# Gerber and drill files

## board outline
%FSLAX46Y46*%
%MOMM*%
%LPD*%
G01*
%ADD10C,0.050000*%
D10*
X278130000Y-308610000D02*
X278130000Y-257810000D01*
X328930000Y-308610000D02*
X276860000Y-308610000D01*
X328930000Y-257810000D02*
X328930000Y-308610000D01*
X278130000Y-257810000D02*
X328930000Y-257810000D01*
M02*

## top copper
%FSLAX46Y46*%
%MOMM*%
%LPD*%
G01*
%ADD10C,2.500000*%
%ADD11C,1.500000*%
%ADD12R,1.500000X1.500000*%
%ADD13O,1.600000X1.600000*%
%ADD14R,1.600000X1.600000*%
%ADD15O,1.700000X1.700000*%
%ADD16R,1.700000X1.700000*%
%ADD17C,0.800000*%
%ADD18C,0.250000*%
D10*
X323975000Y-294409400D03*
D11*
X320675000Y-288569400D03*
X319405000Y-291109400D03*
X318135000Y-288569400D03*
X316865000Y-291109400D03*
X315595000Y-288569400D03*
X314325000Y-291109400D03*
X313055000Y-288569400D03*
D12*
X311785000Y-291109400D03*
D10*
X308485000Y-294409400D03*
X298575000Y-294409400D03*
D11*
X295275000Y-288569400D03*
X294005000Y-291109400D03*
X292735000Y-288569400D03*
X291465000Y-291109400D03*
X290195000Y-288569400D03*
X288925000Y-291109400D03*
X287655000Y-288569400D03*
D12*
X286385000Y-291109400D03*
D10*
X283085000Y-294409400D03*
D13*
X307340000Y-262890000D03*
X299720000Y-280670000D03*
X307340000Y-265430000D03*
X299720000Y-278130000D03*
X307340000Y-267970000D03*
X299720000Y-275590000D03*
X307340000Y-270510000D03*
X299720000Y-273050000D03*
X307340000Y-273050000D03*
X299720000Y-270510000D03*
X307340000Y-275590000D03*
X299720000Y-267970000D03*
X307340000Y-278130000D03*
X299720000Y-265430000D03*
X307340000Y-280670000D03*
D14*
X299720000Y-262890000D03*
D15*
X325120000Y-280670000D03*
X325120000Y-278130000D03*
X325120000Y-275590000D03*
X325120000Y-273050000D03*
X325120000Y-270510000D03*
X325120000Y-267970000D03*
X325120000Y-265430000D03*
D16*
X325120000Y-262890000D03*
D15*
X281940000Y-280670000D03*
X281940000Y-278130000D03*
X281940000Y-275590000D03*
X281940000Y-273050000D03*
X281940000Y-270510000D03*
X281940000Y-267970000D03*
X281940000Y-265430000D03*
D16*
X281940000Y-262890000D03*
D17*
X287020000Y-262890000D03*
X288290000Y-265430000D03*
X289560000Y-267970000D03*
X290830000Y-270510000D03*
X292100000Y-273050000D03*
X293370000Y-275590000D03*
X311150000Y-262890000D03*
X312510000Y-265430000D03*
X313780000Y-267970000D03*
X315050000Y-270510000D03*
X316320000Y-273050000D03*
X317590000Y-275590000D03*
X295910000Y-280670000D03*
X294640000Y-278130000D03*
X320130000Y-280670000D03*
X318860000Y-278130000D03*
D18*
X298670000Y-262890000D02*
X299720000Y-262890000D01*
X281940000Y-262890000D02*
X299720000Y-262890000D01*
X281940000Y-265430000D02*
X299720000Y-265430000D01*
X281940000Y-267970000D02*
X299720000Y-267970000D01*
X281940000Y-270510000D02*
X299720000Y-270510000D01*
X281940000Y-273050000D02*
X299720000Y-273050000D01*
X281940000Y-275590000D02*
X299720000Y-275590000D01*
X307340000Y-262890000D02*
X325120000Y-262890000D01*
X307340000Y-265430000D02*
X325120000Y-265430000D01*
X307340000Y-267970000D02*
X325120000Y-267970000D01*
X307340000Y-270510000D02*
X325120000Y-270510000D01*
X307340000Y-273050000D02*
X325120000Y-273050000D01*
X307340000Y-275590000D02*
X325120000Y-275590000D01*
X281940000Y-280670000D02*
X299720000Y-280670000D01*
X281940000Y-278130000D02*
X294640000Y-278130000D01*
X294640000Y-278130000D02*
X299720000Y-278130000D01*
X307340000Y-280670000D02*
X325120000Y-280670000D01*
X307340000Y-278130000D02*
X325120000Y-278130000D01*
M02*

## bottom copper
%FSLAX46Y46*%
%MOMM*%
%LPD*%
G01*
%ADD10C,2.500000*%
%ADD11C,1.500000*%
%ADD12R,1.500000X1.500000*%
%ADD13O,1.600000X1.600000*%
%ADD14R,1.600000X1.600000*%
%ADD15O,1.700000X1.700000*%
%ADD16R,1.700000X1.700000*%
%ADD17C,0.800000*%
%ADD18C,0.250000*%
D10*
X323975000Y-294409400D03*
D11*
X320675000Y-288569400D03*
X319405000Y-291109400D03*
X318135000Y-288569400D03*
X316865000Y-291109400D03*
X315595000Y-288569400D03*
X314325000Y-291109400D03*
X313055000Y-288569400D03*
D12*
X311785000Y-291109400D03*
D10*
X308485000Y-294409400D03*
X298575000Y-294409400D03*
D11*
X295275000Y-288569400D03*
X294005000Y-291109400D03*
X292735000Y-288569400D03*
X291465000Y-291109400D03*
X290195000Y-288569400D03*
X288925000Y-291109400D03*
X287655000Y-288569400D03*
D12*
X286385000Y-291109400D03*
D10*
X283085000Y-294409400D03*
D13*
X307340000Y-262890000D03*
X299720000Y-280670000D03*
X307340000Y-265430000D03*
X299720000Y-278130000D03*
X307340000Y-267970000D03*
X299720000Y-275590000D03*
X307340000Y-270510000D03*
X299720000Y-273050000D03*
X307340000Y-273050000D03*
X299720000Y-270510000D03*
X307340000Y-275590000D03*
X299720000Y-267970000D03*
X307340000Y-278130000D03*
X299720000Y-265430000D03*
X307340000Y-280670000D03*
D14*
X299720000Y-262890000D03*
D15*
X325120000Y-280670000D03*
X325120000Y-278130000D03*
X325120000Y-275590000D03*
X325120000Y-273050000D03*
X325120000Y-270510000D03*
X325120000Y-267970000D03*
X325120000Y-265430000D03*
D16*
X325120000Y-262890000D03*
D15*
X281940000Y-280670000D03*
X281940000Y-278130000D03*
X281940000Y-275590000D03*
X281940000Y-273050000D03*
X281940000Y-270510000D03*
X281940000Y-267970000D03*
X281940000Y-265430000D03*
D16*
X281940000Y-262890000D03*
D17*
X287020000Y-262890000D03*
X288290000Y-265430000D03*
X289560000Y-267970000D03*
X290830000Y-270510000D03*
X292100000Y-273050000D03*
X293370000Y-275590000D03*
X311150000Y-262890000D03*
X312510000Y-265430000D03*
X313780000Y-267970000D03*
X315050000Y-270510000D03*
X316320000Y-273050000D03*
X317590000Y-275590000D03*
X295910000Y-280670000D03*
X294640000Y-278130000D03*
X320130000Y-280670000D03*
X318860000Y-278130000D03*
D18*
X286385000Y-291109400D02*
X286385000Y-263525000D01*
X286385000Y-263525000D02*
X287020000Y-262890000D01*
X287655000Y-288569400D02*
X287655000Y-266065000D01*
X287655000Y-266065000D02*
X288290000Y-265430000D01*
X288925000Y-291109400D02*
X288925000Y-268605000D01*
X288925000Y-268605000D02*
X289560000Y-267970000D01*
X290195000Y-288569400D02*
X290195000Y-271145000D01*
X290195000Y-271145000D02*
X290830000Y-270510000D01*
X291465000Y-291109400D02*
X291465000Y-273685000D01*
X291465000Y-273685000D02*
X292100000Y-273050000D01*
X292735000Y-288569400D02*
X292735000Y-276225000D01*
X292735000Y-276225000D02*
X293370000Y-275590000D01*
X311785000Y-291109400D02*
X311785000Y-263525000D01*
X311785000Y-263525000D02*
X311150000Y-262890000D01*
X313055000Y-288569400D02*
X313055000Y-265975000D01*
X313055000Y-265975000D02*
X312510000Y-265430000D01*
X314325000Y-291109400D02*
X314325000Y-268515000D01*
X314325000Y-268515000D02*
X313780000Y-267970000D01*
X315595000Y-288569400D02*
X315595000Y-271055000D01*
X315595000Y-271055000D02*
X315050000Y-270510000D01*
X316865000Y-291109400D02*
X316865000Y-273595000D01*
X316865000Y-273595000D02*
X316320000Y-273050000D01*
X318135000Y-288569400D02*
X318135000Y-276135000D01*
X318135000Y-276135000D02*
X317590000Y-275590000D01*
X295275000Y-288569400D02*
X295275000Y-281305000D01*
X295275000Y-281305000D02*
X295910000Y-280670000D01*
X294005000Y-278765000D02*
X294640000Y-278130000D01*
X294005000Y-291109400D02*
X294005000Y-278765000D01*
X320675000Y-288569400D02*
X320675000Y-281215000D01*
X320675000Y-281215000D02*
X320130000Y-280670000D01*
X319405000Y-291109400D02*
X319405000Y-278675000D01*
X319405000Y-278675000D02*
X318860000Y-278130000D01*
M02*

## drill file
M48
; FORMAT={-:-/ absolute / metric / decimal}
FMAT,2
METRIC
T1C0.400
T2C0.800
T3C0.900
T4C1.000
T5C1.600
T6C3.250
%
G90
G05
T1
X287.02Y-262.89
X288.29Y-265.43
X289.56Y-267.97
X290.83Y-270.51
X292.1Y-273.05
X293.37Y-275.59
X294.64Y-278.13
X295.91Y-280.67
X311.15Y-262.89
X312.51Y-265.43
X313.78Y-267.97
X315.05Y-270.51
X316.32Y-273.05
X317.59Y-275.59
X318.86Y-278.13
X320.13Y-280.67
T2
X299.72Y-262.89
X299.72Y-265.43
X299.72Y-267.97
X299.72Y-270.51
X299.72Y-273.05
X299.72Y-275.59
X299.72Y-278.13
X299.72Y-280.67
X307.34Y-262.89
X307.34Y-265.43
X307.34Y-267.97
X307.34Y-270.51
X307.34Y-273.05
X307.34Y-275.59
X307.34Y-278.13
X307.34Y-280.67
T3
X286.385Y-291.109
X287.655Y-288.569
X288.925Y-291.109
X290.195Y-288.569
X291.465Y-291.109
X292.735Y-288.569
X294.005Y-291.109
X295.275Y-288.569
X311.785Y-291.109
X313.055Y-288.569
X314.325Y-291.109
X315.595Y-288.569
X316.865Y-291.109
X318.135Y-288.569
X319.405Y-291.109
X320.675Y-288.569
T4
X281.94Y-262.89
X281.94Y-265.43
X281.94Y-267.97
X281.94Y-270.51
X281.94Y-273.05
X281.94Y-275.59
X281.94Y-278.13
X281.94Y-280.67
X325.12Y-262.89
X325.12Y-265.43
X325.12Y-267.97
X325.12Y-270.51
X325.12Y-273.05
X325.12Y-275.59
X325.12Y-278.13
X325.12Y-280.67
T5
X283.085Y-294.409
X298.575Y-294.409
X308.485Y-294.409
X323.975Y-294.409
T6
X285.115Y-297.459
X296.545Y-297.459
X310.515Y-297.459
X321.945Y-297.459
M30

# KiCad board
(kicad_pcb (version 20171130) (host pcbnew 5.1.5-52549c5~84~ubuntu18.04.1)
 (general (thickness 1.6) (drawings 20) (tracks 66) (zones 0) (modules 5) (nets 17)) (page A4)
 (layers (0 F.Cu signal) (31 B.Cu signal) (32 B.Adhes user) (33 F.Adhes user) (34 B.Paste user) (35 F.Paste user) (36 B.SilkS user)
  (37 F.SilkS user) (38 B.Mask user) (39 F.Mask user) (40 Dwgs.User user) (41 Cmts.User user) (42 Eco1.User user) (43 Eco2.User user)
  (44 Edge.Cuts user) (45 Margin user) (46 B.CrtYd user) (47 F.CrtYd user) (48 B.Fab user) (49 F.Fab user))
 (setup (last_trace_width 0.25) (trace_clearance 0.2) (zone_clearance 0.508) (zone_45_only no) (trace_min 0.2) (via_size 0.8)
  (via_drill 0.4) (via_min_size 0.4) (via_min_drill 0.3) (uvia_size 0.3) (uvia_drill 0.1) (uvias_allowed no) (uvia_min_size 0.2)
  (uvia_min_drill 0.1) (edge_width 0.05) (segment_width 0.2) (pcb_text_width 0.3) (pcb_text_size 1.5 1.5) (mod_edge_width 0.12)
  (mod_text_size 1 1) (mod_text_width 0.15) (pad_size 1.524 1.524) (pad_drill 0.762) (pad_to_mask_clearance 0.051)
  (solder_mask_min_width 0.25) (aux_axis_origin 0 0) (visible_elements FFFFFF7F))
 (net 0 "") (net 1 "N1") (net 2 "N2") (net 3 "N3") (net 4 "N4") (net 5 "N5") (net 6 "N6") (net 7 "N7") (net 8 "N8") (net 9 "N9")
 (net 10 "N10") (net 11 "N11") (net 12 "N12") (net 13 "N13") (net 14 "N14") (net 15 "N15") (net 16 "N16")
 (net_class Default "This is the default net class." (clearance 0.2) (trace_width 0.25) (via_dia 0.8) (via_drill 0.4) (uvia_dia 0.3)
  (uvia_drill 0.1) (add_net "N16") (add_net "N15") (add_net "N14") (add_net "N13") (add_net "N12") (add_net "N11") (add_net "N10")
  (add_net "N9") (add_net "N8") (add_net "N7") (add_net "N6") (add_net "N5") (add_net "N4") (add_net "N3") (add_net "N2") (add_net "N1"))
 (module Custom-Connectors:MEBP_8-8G (layer F.Cu) (at 316.23 306.07 180)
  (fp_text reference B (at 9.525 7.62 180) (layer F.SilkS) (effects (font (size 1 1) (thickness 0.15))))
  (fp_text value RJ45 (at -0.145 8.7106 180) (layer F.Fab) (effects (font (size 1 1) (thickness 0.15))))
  (pad 9 thru_hole circle (at -7.745 11.6606) (size 2.5 2.5) (drill 1.6) (layers *.Cu *.Mask))
  (pad 8 thru_hole circle (at -4.445 17.5006) (size 1.5 1.5) (drill 0.9) (layers *.Cu *.Mask) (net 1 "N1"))
  (pad 7 thru_hole circle (at -3.175 14.9606) (size 1.5 1.5) (drill 0.9) (layers *.Cu *.Mask) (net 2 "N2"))
  (pad 6 thru_hole circle (at -1.905 17.5006) (size 1.5 1.5) (drill 0.9) (layers *.Cu *.Mask) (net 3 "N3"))
  (pad 5 thru_hole circle (at -0.635 14.9606) (size 1.5 1.5) (drill 0.9) (layers *.Cu *.Mask) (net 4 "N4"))
  (pad 4 thru_hole circle (at 0.635 17.5006) (size 1.5 1.5) (drill 0.9) (layers *.Cu *.Mask) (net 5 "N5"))
  (pad 3 thru_hole circle (at 1.905 14.9606) (size 1.5 1.5) (drill 0.9) (layers *.Cu *.Mask) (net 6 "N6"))
  (pad 2 thru_hole circle (at 3.175 17.5006) (size 1.5 1.5) (drill 0.9) (layers *.Cu *.Mask) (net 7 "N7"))
  (pad 1 thru_hole rect (at 4.445 14.9606) (size 1.5 1.5) (drill 0.9) (layers *.Cu *.Mask) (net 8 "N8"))
  (pad "" np_thru_hole circle (at 5.715 8.6106) (size 3.25 3.25) (drill 3.25) (layers *.Cu *.SilkS *.Mask))
  (pad "" np_thru_hole circle (at -5.715 8.6106) (size 3.25 3.25) (drill 3.25) (layers *.Cu *.SilkS *.Mask))
  (pad 9 thru_hole circle (at 7.745 11.6606) (size 2.5 2.5) (drill 1.6) (layers *.Cu *.Mask)))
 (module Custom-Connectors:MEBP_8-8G (layer F.Cu) (at 290.83 306.07 180)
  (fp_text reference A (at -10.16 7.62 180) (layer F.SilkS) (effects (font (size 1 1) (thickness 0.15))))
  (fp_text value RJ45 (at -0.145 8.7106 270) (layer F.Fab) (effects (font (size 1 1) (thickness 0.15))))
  (pad 9 thru_hole circle (at -7.745 11.6606) (size 2.5 2.5) (drill 1.6) (layers *.Cu *.Mask))
  (pad 8 thru_hole circle (at -4.445 17.5006) (size 1.5 1.5) (drill 0.9) (layers *.Cu *.Mask) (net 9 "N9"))
  (pad 7 thru_hole circle (at -3.175 14.9606) (size 1.5 1.5) (drill 0.9) (layers *.Cu *.Mask) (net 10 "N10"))
  (pad 6 thru_hole circle (at -1.905 17.5006) (size 1.5 1.5) (drill 0.9) (layers *.Cu *.Mask) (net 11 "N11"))
  (pad 5 thru_hole circle (at -0.635 14.9606) (size 1.5 1.5) (drill 0.9) (layers *.Cu *.Mask) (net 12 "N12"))
  (pad 4 thru_hole circle (at 0.635 17.5006) (size 1.5 1.5) (drill 0.9) (layers *.Cu *.Mask) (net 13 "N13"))
  (pad 3 thru_hole circle (at 1.905 14.9606) (size 1.5 1.5) (drill 0.9) (layers *.Cu *.Mask) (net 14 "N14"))
  (pad 2 thru_hole circle (at 3.175 17.5006) (size 1.5 1.5) (drill 0.9) (layers *.Cu *.Mask) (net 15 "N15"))
  (pad 1 thru_hole rect (at 4.445 14.9606) (size 1.5 1.5) (drill 0.9) (layers *.Cu *.Mask) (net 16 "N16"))
  (pad "" np_thru_hole circle (at 5.715 8.6106) (size 3.25 3.25) (drill 3.25) (layers *.Cu *.SilkS *.Mask))
  (pad "" np_thru_hole circle (at -5.715 8.6106) (size 3.25 3.25) (drill 3.25) (layers *.Cu *.SilkS *.Mask))
  (pad 9 thru_hole circle (at 7.745 11.6606) (size 2.5 2.5) (drill 1.6) (layers *.Cu *.Mask)))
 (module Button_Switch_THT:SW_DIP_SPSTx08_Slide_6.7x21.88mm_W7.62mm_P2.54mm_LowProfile (layer F.Cu) (at 299.72 262.89)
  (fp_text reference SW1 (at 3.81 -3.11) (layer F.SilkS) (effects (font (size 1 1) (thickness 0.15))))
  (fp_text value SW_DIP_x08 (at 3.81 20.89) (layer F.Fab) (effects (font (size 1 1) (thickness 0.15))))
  (pad 16 thru_hole oval (at 7.62 0) (size 1.6 1.6) (drill 0.8) (layers *.Cu *.Mask) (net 8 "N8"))
  (pad 8 thru_hole oval (at 0 17.78) (size 1.6 1.6) (drill 0.8) (layers *.Cu *.Mask) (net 9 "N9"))
  (pad 15 thru_hole oval (at 7.62 2.54) (size 1.6 1.6) (drill 0.8) (layers *.Cu *.Mask) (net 7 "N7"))
  (pad 7 thru_hole oval (at 0 15.24) (size 1.6 1.6) (drill 0.8) (layers *.Cu *.Mask) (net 10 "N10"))
  (pad 14 thru_hole oval (at 7.62 5.08) (size 1.6 1.6) (drill 0.8) (layers *.Cu *.Mask) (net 6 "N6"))
  (pad 6 thru_hole oval (at 0 12.7) (size 1.6 1.6) (drill 0.8) (layers *.Cu *.Mask) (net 11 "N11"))
  (pad 13 thru_hole oval (at 7.62 7.62) (size 1.6 1.6) (drill 0.8) (layers *.Cu *.Mask) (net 5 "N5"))
  (pad 5 thru_hole oval (at 0 10.16) (size 1.6 1.6) (drill 0.8) (layers *.Cu *.Mask) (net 12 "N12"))
  (pad 12 thru_hole oval (at 7.62 10.16) (size 1.6 1.6) (drill 0.8) (layers *.Cu *.Mask) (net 4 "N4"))
  (pad 4 thru_hole oval (at 0 7.62) (size 1.6 1.6) (drill 0.8) (layers *.Cu *.Mask) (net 13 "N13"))
  (pad 11 thru_hole oval (at 7.62 12.7) (size 1.6 1.6) (drill 0.8) (layers *.Cu *.Mask) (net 3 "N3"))
  (pad 3 thru_hole oval (at 0 5.08) (size 1.6 1.6) (drill 0.8) (layers *.Cu *.Mask) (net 14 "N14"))
  (pad 10 thru_hole oval (at 7.62 15.24) (size 1.6 1.6) (drill 0.8) (layers *.Cu *.Mask) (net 2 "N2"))
  (pad 2 thru_hole oval (at 0 2.54) (size 1.6 1.6) (drill 0.8) (layers *.Cu *.Mask) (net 15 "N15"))
  (pad 9 thru_hole oval (at 7.62 17.78) (size 1.6 1.6) (drill 0.8) (layers *.Cu *.Mask) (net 1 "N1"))
  (pad 1 thru_hole rect (at 0 0) (size 1.6 1.6) (drill 0.8) (layers *.Cu *.Mask) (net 16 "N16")))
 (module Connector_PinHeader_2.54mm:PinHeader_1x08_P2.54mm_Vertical (layer F.Cu) (at 325.12 262.89)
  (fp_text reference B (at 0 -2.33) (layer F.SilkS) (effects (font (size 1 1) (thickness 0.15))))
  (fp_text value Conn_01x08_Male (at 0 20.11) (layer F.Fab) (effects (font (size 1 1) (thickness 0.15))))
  (pad 8 thru_hole oval (at 0 17.78) (size 1.7 1.7) (drill 1) (layers *.Cu *.Mask) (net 1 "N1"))
  (pad 7 thru_hole oval (at 0 15.24) (size 1.7 1.7) (drill 1) (layers *.Cu *.Mask) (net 2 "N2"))
  (pad 6 thru_hole oval (at 0 12.7) (size 1.7 1.7) (drill 1) (layers *.Cu *.Mask) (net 3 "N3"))
  (pad 5 thru_hole oval (at 0 10.16) (size 1.7 1.7) (drill 1) (layers *.Cu *.Mask) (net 4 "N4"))
  (pad 4 thru_hole oval (at 0 7.62) (size 1.7 1.7) (drill 1) (layers *.Cu *.Mask) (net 5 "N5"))
  (pad 3 thru_hole oval (at 0 5.08) (size 1.7 1.7) (drill 1) (layers *.Cu *.Mask) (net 6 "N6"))
  (pad 2 thru_hole oval (at 0 2.54) (size 1.7 1.7) (drill 1) (layers *.Cu *.Mask) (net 7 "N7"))
  (pad 1 thru_hole rect (at 0 0) (size 1.7 1.7) (drill 1) (layers *.Cu *.Mask) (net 8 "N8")))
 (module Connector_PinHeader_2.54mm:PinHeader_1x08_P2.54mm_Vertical (layer F.Cu) (at 281.94 262.89)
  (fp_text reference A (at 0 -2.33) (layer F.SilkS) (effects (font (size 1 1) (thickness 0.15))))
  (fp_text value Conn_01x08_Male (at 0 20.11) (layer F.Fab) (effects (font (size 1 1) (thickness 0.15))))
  (pad 8 thru_hole oval (at 0 17.78) (size 1.7 1.7) (drill 1) (layers *.Cu *.Mask) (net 9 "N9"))
  (pad 7 thru_hole oval (at 0 15.24) (size 1.7 1.7) (drill 1) (layers *.Cu *.Mask) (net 10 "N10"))
  (pad 6 thru_hole oval (at 0 12.7) (size 1.7 1.7) (drill 1) (layers *.Cu *.Mask) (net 11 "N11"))
  (pad 5 thru_hole oval (at 0 10.16) (size 1.7 1.7) (drill 1) (layers *.Cu *.Mask) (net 12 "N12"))
  (pad 4 thru_hole oval (at 0 7.62) (size 1.7 1.7) (drill 1) (layers *.Cu *.Mask) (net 13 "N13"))
  (pad 3 thru_hole oval (at 0 5.08) (size 1.7 1.7) (drill 1) (layers *.Cu *.Mask) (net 14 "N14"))
  (pad 2 thru_hole oval (at 0 2.54) (size 1.7 1.7) (drill 1) (layers *.Cu *.Mask) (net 15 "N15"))
  (pad 1 thru_hole rect (at 0 0) (size 1.7 1.7) (drill 1) (layers *.Cu *.Mask) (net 16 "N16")))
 (gr_line (start 278.13 308.61) (end 278.13 257.81) (layer Edge.Cuts) (width 0.05))
 (gr_line (start 328.93 308.61) (end 276.86 308.61) (layer Edge.Cuts) (width 0.05))
 (gr_line (start 328.93 257.81) (end 328.93 308.61) (layer Edge.Cuts) (width 0.05))
 (gr_line (start 278.13 257.81) (end 328.93 257.81) (layer Edge.Cuts) (width 0.05))
 (segment (start 298.67 262.89) (end 299.72 262.89) (width 0.25) (layer F.Cu) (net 16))
 (segment (start 281.94 262.89) (end 299.72 262.89) (width 0.25) (layer F.Cu) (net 16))
 (segment (start 286.385 291.1094) (end 286.385 263.525) (width 0.25) (layer B.Cu) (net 16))
 (via (at 287.02 262.89) (size 0.8) (drill 0.4) (layers F.Cu B.Cu) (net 16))
 (segment (start 286.385 263.525) (end 287.02 262.89) (width 0.25) (layer B.Cu) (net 16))
 (segment (start 281.94 265.43) (end 299.72 265.43) (width 0.25) (layer F.Cu) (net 15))
 (via (at 288.29 265.43) (size 0.8) (drill 0.4) (layers F.Cu B.Cu) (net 15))
 (segment (start 287.655 288.5694) (end 287.655 266.065) (width 0.25) (layer B.Cu) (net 15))
 (segment (start 287.655 266.065) (end 288.29 265.43) (width 0.25) (layer B.Cu) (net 15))
 (segment (start 281.94 267.97) (end 299.72 267.97) (width 0.25) (layer F.Cu) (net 14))
 (via (at 289.56 267.97) (size 0.8) (drill 0.4) (layers F.Cu B.Cu) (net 14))
 (segment (start 288.925 291.1094) (end 288.925 268.605) (width 0.25) (layer B.Cu) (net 14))
 (segment (start 288.925 268.605) (end 289.56 267.97) (width 0.25) (layer B.Cu) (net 14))
 (segment (start 281.94 270.51) (end 299.72 270.51) (width 0.25) (layer F.Cu) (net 13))
 (via (at 290.83 270.51) (size 0.8) (drill 0.4) (layers F.Cu B.Cu) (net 13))
 (segment (start 290.195 288.5694) (end 290.195 271.145) (width 0.25) (layer B.Cu) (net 13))
 (segment (start 290.195 271.145) (end 290.83 270.51) (width 0.25) (layer B.Cu) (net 13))
 (segment (start 281.94 273.05) (end 299.72 273.05) (width 0.25) (layer F.Cu) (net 12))
 (via (at 292.1 273.05) (size 0.8) (drill 0.4) (layers F.Cu B.Cu) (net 12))
 (segment (start 291.465 291.1094) (end 291.465 273.685) (width 0.25) (layer B.Cu) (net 12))
 (segment (start 291.465 273.685) (end 292.1 273.05) (width 0.25) (layer B.Cu) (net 12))
 (segment (start 281.94 275.59) (end 299.72 275.59) (width 0.25) (layer F.Cu) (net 11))
 (via (at 293.37 275.59) (size 0.8) (drill 0.4) (layers F.Cu B.Cu) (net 11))
 (segment (start 292.735 288.5694) (end 292.735 276.225) (width 0.25) (layer B.Cu) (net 11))
 (segment (start 292.735 276.225) (end 293.37 275.59) (width 0.25) (layer B.Cu) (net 11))
 (segment (start 307.34 262.89) (end 325.12 262.89) (width 0.25) (layer F.Cu) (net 8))
 (via (at 311.15 262.89) (size 0.8) (drill 0.4) (layers F.Cu B.Cu) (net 8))
 (segment (start 311.785 291.1094) (end 311.785 263.525) (width 0.25) (layer B.Cu) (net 8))
 (segment (start 311.785 263.525) (end 311.15 262.89) (width 0.25) (layer B.Cu) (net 8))
 (segment (start 307.34 265.43) (end 325.12 265.43) (width 0.25) (layer F.Cu) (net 7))
 (via (at 312.51 265.43) (size 0.8) (drill 0.4) (layers F.Cu B.Cu) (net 7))
 (segment (start 313.055 288.5694) (end 313.055 265.975) (width 0.25) (layer B.Cu) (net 7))
 (segment (start 313.055 265.975) (end 312.51 265.43) (width 0.25) (layer B.Cu) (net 7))
 (segment (start 307.34 267.97) (end 325.12 267.97) (width 0.25) (layer F.Cu) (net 6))
 (via (at 313.78 267.97) (size 0.8) (drill 0.4) (layers F.Cu B.Cu) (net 6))
 (segment (start 314.325 291.1094) (end 314.325 268.515) (width 0.25) (layer B.Cu) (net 6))
 (segment (start 314.325 268.515) (end 313.78 267.97) (width 0.25) (layer B.Cu) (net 6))
 (segment (start 307.34 270.51) (end 325.12 270.51) (width 0.25) (layer F.Cu) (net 5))
 (via (at 315.05 270.51) (size 0.8) (drill 0.4) (layers F.Cu B.Cu) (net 5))
 (segment (start 315.595 288.5694) (end 315.595 271.055) (width 0.25) (layer B.Cu) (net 5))
 (segment (start 315.595 271.055) (end 315.05 270.51) (width 0.25) (layer B.Cu) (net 5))
 (segment (start 307.34 273.05) (end 325.12 273.05) (width 0.25) (layer F.Cu) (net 4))
 (via (at 316.32 273.05) (size 0.8) (drill 0.4) (layers F.Cu B.Cu) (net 4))
 (segment (start 316.865 291.1094) (end 316.865 273.595) (width 0.25) (layer B.Cu) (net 4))
 (segment (start 316.865 273.595) (end 316.32 273.05) (width 0.25) (layer B.Cu) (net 4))
 (segment (start 307.34 275.59) (end 325.12 275.59) (width 0.25) (layer F.Cu) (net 3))
 (via (at 317.59 275.59) (size 0.8) (drill 0.4) (layers F.Cu B.Cu) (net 3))
 (segment (start 318.135 288.5694) (end 318.135 276.135) (width 0.25) (layer B.Cu) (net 3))
 (segment (start 318.135 276.135) (end 317.59 275.59) (width 0.25) (layer B.Cu) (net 3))
 (segment (start 281.94 280.67) (end 299.72 280.67) (width 0.25) (layer F.Cu) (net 9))
 (segment (start 295.275 288.5694) (end 295.275 281.305) (width 0.25) (layer B.Cu) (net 9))
 (via (at 295.91 280.67) (size 0.8) (drill 0.4) (layers F.Cu B.Cu) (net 9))
 (segment (start 295.275 281.305) (end 295.91 280.67) (width 0.25) (layer B.Cu) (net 9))
 (via (at 294.64 278.13) (size 0.8) (drill 0.4) (layers F.Cu B.Cu) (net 10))
 (segment (start 294.005 278.765) (end 294.64 278.13) (width 0.25) (layer B.Cu) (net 10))
 (segment (start 294.005 291.1094) (end 294.005 278.765) (width 0.25) (layer B.Cu) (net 10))
 (segment (start 281.94 278.13) (end 294.64 278.13) (width 0.25) (layer F.Cu) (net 10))
 (segment (start 294.64 278.13) (end 299.72 278.13) (width 0.25) (layer F.Cu) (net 10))
 (segment (start 307.34 280.67) (end 325.12 280.67) (width 0.25) (layer F.Cu) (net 1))
 (via (at 320.13 280.67) (size 0.8) (drill 0.4) (layers F.Cu B.Cu) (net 1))
 (segment (start 320.675 288.5694) (end 320.675 281.215) (width 0.25) (layer B.Cu) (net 1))
 (segment (start 320.675 281.215) (end 320.13 280.67) (width 0.25) (layer B.Cu) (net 1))
 (segment (start 307.34 278.13) (end 325.12 278.13) (width 0.25) (layer F.Cu) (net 2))
 (via (at 318.86 278.13) (size 0.8) (drill 0.4) (layers F.Cu B.Cu) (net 2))
 (segment (start 319.405 291.1094) (end 319.405 278.675) (width 0.25) (layer B.Cu) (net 2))
 (segment (start 319.405 278.675) (end 318.86 278.13) (width 0.25) (layer B.Cu) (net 2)))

